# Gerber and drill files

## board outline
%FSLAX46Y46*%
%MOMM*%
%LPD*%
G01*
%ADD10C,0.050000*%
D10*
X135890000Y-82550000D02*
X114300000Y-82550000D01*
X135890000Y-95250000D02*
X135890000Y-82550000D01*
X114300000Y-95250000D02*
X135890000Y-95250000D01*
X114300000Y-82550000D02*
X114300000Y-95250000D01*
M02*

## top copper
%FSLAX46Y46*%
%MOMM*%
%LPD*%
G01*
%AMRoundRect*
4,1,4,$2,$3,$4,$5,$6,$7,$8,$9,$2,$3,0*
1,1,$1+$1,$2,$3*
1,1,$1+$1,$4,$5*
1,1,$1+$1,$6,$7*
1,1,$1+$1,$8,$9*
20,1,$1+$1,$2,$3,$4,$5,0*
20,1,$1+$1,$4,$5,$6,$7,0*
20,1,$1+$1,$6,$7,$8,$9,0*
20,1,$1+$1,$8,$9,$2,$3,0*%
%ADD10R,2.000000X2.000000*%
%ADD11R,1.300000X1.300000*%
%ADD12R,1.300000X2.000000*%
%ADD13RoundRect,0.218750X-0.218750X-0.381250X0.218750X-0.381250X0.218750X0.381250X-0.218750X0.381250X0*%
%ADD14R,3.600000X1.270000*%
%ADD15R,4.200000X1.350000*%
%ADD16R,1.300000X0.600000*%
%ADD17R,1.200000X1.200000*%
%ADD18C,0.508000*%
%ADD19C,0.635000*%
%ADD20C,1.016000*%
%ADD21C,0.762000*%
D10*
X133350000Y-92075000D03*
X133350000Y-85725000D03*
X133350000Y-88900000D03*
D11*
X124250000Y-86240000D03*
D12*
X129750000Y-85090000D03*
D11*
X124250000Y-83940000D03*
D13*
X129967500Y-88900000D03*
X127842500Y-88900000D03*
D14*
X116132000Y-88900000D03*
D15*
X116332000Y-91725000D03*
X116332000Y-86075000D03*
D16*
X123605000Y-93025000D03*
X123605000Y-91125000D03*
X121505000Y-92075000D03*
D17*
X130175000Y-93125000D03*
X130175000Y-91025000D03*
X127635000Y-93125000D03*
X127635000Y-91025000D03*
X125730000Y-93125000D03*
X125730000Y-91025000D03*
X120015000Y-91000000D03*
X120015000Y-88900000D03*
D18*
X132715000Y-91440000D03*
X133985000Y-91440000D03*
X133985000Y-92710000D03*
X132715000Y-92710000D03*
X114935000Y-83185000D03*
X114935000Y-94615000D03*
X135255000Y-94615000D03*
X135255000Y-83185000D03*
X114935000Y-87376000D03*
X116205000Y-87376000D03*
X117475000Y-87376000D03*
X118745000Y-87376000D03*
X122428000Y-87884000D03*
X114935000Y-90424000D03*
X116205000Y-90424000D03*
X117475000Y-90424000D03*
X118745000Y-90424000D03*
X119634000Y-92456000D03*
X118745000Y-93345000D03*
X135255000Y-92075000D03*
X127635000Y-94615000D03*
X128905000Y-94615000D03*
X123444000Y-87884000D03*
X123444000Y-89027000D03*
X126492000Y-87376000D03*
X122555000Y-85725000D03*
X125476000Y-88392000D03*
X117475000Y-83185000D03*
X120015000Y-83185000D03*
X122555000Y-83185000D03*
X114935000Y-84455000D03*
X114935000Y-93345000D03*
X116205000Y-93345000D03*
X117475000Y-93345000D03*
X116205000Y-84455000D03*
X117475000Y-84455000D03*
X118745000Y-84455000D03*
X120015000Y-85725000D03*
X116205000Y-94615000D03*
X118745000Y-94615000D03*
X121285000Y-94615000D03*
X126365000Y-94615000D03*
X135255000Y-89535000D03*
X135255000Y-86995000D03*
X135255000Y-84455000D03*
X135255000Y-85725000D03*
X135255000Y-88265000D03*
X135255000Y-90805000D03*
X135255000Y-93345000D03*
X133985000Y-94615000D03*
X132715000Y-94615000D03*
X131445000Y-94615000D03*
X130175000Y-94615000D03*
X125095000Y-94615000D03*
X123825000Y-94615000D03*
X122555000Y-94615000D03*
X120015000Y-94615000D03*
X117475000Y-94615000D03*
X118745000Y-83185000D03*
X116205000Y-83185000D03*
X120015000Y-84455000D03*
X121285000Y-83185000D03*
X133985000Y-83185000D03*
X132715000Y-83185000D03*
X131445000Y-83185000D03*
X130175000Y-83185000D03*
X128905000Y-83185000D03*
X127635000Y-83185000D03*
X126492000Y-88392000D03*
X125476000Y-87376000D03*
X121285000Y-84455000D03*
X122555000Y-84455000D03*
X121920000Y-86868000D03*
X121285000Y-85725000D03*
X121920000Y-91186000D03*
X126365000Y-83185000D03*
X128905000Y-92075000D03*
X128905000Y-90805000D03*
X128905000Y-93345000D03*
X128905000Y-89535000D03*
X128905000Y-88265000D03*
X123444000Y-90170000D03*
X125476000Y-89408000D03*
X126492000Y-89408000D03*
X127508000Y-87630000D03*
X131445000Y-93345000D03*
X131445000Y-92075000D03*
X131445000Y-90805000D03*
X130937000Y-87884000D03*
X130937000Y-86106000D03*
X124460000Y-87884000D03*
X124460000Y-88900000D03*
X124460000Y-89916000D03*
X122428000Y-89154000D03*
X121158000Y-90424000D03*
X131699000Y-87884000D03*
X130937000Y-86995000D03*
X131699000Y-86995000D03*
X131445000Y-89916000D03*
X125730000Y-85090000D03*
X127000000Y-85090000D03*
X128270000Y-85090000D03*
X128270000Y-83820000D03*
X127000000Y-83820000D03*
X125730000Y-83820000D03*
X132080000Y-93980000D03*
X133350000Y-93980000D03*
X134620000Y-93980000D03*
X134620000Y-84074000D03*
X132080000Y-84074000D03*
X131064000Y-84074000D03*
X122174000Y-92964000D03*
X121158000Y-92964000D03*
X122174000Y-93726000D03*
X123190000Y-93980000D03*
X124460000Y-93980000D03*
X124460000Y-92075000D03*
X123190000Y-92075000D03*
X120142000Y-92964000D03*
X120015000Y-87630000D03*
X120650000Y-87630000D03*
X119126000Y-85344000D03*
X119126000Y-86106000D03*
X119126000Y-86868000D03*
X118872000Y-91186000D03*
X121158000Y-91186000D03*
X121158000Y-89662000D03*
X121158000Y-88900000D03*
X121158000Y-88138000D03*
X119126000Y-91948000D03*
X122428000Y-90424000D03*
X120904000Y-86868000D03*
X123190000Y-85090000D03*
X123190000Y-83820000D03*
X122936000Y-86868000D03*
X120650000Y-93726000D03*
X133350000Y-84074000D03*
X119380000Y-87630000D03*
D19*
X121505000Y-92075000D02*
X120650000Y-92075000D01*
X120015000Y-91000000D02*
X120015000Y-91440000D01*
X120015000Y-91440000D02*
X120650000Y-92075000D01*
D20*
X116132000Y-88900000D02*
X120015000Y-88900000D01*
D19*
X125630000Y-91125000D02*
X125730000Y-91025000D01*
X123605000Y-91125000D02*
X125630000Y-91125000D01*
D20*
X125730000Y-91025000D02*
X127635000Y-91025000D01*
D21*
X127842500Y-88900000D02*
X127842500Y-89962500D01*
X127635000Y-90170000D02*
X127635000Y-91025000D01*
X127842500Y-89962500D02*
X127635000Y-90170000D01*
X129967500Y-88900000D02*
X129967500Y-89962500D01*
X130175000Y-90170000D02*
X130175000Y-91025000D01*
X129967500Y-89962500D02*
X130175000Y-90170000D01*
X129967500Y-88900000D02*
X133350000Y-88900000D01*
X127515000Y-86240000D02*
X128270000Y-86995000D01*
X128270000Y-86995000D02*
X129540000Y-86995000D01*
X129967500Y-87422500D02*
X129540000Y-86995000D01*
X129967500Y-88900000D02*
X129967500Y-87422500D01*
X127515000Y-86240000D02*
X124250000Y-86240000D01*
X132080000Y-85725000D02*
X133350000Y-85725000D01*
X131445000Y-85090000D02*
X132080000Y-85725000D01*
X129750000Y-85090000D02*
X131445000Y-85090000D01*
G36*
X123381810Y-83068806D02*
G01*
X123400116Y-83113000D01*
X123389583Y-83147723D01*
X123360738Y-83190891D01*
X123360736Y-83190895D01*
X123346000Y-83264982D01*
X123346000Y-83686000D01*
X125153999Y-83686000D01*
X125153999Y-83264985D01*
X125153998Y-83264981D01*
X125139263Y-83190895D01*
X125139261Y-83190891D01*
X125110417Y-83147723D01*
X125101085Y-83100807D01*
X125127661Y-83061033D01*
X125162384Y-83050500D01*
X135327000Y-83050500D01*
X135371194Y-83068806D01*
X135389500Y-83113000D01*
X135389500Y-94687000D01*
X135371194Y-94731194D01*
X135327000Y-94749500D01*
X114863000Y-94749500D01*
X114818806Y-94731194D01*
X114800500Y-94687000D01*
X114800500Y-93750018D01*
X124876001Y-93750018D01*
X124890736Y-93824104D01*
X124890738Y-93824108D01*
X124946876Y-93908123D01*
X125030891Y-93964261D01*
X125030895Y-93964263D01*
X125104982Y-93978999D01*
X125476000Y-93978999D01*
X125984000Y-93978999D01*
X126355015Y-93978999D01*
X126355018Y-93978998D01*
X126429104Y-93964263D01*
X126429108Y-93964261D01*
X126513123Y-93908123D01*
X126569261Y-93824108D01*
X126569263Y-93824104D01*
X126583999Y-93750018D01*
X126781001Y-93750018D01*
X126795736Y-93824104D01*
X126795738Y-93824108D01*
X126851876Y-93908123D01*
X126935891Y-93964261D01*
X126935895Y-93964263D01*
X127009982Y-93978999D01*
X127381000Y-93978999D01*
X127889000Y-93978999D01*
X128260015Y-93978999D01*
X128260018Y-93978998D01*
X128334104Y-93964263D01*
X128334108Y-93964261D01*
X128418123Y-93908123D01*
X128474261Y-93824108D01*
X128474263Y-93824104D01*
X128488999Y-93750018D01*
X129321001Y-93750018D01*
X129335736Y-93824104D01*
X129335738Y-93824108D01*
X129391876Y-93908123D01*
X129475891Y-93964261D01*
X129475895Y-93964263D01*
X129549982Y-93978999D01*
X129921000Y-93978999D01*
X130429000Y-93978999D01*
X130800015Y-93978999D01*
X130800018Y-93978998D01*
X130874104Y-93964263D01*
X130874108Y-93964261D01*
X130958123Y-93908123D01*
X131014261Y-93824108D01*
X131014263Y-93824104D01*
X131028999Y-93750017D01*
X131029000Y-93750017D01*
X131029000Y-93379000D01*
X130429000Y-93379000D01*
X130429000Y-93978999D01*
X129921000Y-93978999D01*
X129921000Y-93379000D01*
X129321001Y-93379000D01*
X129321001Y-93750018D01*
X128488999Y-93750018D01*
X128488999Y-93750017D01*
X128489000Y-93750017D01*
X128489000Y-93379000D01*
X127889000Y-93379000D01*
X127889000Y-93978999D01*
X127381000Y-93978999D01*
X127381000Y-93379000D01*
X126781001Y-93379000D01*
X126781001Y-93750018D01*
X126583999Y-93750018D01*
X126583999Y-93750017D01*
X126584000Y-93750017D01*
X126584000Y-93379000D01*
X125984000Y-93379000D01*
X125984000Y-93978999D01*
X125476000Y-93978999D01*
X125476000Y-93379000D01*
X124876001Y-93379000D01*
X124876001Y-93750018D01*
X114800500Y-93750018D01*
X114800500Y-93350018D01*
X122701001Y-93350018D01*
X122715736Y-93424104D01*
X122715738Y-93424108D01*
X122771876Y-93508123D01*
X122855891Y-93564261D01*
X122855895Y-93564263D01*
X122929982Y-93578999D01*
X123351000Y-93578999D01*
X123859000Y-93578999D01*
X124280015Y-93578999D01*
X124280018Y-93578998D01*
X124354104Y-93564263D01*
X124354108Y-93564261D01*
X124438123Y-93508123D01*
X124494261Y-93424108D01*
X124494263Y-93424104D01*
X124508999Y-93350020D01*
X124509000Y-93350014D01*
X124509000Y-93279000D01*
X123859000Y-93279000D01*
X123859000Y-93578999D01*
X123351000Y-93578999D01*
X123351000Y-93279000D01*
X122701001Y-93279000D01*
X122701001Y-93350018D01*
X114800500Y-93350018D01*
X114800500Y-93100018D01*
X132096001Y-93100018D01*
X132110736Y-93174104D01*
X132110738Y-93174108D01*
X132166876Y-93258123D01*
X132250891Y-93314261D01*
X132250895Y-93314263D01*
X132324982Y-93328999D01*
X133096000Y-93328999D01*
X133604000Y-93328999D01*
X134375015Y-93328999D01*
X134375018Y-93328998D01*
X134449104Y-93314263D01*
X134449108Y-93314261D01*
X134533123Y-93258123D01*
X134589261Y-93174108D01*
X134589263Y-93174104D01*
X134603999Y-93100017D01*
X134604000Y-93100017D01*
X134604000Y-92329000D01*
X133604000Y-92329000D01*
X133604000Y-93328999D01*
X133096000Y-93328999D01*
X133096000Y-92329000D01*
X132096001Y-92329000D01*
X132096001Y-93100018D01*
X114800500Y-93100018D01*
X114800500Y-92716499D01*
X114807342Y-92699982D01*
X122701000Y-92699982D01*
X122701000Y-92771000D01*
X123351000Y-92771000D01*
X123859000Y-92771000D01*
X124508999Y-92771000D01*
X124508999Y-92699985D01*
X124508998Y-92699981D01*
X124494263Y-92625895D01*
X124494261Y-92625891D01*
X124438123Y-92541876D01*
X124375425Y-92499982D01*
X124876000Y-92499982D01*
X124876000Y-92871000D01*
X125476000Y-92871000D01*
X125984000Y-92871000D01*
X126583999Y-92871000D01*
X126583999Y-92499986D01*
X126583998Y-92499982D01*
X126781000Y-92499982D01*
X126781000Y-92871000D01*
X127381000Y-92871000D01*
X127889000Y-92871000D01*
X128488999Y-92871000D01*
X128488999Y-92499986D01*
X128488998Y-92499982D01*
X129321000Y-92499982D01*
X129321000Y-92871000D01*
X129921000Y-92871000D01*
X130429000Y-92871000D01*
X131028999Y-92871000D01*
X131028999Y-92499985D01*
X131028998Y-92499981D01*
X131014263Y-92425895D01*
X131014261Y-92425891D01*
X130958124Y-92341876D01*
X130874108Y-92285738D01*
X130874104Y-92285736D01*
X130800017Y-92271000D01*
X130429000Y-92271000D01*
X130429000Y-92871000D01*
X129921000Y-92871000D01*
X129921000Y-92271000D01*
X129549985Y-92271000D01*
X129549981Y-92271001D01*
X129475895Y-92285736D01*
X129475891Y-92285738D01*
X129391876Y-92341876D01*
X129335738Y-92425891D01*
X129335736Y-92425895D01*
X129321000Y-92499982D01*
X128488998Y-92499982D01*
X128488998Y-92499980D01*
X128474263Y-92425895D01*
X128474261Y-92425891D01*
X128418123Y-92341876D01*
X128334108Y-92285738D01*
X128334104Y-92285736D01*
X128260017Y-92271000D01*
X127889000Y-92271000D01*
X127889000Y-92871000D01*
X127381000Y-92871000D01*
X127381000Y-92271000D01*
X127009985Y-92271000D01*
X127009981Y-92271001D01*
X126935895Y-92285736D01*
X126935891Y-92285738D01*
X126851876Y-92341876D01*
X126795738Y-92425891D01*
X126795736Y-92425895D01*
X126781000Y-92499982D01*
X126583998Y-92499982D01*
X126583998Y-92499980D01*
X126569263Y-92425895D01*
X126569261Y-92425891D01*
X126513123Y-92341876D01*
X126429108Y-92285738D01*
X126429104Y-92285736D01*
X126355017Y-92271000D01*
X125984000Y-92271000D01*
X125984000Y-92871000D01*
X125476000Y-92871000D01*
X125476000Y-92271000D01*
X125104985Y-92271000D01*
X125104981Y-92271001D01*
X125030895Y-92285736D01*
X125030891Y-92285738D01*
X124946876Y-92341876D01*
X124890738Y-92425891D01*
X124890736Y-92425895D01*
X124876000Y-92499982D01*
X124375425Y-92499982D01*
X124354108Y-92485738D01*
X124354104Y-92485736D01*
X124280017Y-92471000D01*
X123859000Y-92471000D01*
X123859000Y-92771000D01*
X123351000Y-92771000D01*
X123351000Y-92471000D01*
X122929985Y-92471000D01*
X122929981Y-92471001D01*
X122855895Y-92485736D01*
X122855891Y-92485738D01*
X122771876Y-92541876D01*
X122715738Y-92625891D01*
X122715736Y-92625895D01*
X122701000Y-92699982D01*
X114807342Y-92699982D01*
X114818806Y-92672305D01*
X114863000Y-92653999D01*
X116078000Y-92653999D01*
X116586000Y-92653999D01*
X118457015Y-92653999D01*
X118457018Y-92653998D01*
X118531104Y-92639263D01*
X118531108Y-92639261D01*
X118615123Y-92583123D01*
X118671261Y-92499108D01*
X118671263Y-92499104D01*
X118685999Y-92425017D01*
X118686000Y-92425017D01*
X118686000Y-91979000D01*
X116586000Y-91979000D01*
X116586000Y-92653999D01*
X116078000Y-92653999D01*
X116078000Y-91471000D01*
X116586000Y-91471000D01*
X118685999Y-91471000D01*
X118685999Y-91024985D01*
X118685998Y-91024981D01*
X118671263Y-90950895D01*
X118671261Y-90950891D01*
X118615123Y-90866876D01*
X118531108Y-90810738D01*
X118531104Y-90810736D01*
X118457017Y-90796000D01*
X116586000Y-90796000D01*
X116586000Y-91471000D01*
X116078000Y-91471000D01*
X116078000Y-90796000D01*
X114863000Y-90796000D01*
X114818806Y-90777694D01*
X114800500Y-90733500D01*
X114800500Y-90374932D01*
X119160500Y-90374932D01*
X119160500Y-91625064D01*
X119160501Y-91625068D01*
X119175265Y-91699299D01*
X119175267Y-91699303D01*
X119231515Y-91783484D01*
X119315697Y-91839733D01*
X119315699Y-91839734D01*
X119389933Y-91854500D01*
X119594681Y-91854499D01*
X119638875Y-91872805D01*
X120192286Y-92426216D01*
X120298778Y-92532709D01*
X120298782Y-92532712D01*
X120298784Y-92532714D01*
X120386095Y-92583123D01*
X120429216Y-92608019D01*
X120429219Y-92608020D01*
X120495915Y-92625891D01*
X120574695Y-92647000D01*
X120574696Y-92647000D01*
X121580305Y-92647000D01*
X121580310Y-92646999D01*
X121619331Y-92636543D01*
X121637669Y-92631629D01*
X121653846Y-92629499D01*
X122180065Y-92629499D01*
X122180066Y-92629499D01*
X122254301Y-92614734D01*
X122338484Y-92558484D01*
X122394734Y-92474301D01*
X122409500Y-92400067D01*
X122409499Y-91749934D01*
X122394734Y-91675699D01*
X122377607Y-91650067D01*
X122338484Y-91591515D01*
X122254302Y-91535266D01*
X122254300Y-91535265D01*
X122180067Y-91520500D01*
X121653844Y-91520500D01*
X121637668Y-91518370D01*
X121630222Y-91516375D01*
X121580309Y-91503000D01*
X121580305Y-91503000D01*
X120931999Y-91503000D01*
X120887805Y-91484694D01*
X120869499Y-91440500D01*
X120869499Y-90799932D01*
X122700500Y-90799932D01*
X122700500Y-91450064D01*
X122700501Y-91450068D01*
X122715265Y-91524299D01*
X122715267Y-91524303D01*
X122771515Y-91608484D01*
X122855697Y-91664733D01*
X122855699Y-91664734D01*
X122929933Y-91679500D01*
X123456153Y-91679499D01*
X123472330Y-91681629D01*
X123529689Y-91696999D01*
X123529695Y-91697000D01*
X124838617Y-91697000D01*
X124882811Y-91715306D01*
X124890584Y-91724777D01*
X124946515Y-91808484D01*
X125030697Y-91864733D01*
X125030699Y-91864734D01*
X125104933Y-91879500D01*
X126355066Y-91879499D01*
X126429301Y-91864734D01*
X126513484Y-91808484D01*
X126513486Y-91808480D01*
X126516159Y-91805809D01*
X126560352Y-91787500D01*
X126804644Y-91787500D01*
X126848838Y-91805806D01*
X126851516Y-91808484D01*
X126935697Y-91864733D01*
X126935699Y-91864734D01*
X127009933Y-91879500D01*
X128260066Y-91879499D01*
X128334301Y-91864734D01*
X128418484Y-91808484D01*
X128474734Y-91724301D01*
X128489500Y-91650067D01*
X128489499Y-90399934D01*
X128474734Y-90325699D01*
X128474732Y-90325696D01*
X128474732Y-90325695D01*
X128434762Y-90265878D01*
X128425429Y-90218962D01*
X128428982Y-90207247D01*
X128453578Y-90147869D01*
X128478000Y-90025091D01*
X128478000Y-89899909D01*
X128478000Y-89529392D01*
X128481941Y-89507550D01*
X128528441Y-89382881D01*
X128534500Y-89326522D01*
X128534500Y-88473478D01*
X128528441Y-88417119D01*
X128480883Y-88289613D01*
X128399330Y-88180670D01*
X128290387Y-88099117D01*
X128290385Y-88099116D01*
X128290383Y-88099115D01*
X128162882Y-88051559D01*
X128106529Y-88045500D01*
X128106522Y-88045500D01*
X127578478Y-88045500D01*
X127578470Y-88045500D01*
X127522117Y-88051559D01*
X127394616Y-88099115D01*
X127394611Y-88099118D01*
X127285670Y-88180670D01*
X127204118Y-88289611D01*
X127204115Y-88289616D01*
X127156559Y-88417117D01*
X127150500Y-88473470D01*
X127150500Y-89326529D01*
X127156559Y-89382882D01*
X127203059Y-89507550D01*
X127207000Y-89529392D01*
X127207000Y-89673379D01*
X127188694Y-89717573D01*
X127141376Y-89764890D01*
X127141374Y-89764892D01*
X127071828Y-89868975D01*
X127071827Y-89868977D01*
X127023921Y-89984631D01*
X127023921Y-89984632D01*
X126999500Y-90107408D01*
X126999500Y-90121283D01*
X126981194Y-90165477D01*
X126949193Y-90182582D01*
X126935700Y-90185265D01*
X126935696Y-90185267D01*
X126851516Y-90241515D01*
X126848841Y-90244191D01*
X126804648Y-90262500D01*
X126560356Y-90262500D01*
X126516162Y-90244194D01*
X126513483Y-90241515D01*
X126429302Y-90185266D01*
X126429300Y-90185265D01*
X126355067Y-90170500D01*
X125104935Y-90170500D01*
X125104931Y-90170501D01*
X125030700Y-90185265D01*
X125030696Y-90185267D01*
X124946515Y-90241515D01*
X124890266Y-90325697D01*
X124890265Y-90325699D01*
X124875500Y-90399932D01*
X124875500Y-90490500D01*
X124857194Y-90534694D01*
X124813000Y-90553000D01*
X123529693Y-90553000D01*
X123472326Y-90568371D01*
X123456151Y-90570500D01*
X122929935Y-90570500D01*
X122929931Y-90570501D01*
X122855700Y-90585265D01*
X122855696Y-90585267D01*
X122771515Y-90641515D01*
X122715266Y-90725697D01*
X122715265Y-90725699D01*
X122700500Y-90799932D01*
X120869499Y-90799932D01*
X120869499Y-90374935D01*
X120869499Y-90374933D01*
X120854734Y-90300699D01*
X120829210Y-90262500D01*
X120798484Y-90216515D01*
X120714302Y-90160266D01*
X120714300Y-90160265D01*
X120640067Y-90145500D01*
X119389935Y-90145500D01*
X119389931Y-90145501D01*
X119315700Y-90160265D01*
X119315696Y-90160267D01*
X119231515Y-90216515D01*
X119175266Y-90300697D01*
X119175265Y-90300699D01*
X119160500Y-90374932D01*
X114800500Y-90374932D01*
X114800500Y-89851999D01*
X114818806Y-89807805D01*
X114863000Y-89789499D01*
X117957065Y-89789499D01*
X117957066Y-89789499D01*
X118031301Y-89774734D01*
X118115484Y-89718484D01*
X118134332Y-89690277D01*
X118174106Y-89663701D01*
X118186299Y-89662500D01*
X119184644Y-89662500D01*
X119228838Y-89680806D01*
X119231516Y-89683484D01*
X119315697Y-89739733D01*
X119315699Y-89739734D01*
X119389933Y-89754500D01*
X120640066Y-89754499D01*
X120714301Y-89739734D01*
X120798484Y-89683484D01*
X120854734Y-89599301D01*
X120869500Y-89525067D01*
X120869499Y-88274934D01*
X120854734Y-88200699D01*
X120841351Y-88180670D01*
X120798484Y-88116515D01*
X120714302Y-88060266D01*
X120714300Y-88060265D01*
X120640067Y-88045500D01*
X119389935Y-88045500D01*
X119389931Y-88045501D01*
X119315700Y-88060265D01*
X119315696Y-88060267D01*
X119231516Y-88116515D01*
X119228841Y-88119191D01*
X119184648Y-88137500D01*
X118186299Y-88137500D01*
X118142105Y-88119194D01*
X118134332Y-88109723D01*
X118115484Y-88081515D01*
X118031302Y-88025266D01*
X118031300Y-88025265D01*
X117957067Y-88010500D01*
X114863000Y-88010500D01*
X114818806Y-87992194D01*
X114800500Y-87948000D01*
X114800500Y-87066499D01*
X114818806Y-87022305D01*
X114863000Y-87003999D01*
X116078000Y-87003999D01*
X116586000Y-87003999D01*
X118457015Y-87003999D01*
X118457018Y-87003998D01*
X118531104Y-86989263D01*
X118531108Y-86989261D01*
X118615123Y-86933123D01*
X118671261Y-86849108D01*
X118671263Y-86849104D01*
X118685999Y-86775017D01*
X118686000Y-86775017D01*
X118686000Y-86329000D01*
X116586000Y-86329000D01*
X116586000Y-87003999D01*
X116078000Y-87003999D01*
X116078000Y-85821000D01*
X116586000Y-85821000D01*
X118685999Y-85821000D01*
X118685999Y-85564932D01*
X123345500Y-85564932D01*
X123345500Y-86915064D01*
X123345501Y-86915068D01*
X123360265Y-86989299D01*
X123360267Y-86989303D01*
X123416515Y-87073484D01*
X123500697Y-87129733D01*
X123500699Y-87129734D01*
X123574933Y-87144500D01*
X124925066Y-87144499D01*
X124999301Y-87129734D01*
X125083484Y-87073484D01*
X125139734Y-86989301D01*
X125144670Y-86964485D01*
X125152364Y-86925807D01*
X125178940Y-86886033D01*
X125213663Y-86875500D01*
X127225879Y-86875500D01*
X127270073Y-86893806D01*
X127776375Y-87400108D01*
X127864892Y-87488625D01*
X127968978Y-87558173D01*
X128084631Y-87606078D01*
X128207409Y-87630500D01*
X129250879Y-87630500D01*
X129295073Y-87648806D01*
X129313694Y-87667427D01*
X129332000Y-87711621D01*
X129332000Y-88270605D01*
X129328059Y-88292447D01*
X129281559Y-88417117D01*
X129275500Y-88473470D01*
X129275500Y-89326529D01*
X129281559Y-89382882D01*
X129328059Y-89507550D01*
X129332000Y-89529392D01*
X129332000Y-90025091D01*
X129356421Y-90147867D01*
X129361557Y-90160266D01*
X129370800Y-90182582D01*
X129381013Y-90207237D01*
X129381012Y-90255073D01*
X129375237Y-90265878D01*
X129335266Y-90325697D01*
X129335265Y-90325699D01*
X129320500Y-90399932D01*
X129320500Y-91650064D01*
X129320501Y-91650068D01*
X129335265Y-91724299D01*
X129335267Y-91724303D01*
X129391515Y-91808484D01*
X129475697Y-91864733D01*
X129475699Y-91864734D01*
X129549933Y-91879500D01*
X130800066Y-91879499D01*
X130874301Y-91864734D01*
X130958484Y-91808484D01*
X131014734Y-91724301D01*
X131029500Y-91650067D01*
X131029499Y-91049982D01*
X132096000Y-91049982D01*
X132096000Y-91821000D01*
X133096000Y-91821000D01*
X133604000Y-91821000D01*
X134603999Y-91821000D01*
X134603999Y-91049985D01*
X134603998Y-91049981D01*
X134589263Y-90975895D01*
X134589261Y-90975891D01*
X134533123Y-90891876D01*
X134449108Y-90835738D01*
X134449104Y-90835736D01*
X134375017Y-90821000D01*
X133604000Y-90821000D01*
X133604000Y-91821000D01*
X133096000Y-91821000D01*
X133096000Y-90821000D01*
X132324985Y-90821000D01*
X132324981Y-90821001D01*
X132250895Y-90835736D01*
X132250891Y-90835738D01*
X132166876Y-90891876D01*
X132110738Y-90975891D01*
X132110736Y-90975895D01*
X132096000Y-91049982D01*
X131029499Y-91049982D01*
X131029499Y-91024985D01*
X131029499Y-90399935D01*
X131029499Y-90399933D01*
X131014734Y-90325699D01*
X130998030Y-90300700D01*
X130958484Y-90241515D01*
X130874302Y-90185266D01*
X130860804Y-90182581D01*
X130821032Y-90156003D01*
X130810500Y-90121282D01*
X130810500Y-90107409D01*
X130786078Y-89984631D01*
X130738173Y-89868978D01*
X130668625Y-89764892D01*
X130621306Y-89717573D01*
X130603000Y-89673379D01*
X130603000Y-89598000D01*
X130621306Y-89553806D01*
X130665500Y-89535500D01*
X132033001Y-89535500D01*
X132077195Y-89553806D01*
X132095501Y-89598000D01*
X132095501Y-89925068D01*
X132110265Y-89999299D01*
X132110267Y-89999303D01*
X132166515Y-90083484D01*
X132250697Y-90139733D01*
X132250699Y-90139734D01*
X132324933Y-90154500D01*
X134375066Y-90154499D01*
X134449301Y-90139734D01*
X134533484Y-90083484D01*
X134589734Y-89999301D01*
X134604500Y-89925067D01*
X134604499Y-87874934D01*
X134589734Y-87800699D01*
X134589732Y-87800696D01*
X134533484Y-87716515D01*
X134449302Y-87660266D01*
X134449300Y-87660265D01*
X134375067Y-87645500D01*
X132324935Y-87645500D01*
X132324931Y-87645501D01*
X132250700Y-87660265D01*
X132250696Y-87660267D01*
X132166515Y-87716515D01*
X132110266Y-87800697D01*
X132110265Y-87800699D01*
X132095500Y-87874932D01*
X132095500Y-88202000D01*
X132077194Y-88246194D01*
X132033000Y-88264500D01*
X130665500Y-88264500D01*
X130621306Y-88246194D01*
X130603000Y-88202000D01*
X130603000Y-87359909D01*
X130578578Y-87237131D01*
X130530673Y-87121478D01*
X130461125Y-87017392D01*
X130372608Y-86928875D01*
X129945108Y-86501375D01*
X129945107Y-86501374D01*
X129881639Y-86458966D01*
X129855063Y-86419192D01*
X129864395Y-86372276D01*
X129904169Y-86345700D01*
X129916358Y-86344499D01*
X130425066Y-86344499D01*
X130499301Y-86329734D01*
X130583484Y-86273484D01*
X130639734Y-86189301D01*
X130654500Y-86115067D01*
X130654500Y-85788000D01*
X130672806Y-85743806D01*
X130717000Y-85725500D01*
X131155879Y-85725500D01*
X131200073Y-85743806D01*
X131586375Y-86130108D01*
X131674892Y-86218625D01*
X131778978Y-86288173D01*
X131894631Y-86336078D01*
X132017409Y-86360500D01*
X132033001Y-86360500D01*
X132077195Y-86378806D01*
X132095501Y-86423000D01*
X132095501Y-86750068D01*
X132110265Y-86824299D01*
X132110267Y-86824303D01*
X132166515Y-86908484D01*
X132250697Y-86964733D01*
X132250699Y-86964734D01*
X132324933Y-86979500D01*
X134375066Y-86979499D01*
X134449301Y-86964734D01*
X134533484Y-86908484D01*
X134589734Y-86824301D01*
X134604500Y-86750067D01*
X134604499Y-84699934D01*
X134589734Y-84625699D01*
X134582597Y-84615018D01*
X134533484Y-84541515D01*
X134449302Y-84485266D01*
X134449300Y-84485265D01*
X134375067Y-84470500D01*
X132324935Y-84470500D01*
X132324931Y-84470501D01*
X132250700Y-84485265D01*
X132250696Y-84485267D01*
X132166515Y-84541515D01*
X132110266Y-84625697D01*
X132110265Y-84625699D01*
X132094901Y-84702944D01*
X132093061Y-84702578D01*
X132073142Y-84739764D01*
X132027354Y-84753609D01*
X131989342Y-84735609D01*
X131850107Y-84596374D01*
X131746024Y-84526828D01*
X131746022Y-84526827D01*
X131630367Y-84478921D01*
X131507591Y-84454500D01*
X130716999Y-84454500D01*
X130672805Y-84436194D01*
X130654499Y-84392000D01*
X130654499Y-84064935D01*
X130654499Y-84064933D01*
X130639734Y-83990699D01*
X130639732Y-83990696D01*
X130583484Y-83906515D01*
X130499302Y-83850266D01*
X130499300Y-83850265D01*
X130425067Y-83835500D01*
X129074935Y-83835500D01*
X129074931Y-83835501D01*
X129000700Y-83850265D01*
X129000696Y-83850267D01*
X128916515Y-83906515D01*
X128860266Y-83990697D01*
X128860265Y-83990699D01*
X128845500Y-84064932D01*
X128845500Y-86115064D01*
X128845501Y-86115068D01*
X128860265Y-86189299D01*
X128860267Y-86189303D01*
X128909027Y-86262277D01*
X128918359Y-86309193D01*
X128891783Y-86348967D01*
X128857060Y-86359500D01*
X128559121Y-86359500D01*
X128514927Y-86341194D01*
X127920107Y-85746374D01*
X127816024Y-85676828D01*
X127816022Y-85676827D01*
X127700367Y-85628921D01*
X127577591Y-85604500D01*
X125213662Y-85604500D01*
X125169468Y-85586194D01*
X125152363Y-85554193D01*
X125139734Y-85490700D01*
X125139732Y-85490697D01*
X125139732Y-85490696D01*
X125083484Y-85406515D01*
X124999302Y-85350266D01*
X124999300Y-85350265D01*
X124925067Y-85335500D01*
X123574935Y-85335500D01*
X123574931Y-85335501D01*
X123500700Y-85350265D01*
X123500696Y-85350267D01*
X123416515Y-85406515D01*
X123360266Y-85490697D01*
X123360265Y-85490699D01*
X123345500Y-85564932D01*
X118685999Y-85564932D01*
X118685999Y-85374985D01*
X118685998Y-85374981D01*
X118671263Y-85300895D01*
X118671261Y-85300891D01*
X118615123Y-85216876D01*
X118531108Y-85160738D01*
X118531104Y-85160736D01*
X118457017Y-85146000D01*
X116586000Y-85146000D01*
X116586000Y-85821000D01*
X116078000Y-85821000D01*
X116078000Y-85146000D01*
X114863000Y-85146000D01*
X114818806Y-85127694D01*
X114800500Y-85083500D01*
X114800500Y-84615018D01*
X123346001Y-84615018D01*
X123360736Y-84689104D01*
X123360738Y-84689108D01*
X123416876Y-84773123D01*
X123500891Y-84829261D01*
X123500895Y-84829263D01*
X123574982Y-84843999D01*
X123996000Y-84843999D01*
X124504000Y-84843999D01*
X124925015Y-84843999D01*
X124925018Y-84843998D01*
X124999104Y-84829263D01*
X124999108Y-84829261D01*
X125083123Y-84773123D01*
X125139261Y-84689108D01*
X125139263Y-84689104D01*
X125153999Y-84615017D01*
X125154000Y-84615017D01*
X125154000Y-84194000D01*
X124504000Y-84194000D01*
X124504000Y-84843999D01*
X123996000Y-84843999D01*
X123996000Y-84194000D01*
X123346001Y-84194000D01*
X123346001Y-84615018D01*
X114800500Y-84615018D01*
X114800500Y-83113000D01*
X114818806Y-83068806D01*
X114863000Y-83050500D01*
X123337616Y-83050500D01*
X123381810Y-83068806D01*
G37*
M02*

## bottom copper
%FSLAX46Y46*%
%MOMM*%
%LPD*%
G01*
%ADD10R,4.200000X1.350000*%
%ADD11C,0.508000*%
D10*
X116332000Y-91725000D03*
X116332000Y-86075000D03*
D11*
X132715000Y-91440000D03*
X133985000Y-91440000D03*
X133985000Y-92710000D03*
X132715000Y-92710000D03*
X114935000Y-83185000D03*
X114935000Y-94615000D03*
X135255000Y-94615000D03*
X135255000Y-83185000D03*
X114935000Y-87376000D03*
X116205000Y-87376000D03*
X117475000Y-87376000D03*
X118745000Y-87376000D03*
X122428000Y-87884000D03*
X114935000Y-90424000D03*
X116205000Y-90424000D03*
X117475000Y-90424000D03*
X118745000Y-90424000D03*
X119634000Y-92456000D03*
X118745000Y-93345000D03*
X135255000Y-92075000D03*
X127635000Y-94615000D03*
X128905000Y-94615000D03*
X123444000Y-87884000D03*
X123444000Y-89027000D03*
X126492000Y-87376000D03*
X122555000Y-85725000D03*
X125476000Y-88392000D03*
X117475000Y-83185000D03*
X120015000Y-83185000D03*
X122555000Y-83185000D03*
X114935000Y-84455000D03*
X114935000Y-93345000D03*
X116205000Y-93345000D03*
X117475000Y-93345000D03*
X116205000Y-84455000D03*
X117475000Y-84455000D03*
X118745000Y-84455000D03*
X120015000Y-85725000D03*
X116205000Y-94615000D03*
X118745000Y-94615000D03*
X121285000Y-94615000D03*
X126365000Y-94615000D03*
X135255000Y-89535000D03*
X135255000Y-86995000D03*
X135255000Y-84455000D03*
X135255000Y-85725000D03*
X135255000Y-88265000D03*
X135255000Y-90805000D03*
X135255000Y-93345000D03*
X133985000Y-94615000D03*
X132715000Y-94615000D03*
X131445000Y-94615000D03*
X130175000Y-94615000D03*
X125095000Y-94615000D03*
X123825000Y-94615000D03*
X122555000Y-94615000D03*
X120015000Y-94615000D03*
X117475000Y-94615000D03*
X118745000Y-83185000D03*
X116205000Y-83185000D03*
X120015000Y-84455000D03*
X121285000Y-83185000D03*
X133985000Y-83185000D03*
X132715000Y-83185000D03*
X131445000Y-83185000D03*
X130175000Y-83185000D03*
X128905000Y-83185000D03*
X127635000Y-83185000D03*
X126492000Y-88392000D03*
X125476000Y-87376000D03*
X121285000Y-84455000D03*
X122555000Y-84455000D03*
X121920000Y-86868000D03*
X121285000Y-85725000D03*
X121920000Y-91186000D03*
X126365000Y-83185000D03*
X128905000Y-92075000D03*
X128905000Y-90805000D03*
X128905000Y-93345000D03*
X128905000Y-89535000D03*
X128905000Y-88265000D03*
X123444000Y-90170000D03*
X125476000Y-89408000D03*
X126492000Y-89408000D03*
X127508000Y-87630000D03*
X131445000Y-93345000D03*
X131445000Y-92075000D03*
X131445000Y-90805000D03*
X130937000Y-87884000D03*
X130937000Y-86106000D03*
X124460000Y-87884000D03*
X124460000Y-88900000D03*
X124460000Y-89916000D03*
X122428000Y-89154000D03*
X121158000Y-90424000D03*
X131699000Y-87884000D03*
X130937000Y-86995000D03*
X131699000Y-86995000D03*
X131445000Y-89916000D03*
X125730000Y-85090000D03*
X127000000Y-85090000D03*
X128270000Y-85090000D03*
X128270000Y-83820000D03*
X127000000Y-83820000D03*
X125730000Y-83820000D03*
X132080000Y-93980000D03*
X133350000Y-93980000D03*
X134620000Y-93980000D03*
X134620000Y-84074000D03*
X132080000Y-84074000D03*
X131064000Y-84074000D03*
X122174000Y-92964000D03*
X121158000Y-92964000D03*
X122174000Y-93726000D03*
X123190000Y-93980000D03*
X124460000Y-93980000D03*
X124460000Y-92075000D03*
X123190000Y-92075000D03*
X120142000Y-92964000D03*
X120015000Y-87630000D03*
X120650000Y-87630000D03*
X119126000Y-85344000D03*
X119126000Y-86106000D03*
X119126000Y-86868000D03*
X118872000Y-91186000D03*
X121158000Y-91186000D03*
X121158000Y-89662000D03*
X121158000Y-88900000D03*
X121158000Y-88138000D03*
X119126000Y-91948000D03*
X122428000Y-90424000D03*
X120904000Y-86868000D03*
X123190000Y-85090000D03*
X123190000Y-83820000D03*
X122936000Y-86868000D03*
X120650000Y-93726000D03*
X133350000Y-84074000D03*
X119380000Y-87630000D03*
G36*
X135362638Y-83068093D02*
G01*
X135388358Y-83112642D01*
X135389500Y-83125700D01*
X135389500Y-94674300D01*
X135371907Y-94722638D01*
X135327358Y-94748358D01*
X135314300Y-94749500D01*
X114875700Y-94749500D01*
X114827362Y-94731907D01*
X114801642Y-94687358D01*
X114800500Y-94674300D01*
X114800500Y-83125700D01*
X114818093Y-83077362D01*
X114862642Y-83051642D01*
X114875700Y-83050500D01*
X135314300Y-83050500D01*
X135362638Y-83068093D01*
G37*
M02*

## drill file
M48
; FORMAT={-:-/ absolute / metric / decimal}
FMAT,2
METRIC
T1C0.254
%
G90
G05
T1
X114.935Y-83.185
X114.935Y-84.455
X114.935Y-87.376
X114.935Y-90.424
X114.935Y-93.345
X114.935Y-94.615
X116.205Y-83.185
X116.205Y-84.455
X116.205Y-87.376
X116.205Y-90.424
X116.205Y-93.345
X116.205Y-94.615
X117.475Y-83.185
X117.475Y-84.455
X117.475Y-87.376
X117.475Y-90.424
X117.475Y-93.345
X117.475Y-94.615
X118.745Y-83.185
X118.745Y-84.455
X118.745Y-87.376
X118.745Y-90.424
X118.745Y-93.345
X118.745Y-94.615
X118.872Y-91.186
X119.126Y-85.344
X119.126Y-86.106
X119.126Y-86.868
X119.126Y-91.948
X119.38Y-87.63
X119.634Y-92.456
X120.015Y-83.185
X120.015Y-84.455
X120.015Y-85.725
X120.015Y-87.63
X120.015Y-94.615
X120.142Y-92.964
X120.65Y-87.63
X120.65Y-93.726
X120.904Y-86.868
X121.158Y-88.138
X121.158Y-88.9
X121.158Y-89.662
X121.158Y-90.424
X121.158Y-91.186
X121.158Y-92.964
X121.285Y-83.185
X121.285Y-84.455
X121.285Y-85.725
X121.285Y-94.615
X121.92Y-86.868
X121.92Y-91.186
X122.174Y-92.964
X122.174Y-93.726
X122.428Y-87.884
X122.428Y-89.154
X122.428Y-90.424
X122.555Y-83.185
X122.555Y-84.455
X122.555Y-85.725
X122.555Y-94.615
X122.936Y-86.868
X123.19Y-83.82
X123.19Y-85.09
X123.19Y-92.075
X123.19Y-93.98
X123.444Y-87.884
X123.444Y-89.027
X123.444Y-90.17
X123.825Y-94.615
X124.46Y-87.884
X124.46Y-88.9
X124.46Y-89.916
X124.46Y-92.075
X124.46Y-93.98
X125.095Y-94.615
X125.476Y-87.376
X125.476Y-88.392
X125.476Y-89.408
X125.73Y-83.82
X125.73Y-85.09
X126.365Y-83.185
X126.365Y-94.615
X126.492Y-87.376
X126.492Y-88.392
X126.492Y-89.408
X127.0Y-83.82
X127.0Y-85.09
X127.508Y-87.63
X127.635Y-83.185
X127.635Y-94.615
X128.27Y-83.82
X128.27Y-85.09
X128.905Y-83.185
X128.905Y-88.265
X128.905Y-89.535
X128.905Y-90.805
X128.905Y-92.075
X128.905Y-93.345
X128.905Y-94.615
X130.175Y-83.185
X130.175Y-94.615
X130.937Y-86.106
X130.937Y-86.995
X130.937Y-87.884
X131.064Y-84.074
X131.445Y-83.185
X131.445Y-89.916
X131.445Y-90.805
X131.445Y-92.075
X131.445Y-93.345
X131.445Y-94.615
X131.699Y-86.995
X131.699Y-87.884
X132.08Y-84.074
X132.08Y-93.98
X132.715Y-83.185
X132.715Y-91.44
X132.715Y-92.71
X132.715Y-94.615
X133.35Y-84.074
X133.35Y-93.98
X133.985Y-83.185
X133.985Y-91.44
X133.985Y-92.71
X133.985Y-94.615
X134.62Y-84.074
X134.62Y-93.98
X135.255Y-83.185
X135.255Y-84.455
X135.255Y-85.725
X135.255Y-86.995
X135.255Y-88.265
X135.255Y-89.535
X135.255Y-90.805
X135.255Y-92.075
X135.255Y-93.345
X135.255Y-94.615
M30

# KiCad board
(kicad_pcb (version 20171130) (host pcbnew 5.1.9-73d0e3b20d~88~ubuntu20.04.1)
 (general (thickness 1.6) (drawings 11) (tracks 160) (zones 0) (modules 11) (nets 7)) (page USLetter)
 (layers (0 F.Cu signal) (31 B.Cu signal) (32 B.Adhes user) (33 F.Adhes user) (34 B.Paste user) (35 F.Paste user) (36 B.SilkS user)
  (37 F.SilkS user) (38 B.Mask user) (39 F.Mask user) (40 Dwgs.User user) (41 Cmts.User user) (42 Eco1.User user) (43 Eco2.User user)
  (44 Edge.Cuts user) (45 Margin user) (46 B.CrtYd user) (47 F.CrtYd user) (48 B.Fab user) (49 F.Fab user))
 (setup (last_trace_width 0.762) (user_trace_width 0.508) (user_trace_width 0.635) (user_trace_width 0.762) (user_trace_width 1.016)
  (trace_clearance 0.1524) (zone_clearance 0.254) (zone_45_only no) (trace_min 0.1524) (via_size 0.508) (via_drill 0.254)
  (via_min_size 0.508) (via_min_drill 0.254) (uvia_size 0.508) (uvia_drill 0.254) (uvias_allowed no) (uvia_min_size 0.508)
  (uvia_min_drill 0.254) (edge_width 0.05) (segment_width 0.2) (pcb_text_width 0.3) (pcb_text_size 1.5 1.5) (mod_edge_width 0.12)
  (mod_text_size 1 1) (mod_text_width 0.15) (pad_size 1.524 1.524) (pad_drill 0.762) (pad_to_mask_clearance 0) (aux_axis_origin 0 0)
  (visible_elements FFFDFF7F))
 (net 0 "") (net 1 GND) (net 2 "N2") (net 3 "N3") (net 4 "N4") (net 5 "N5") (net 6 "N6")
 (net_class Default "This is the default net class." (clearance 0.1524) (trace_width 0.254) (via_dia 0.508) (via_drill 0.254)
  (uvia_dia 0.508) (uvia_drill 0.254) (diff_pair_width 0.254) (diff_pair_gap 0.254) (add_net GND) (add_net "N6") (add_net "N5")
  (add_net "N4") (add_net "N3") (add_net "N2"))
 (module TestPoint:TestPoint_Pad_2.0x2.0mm (layer F.Cu) (at 133.35 92.075 270)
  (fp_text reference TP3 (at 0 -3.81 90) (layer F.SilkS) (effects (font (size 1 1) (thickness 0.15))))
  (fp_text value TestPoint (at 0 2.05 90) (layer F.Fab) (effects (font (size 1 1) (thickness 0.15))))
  (pad 1 smd rect (at 0 0 270) (size 2 2) (layers F.Cu F.Mask) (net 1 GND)))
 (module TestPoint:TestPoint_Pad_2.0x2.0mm (layer F.Cu) (at 133.35 85.725 270)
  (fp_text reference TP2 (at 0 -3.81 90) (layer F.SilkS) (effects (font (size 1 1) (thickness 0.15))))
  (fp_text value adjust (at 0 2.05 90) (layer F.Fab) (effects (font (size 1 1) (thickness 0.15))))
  (pad 1 smd rect (at 0 0 270) (size 2 2) (layers F.Cu F.Mask) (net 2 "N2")))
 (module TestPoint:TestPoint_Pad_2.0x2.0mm (layer F.Cu) (at 133.35 88.9 270)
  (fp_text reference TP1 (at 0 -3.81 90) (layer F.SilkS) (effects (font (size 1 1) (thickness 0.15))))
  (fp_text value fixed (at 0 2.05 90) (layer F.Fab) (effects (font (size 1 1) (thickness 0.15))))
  (pad 1 smd rect (at 0 0 270) (size 2 2) (layers F.Cu F.Mask) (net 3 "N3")))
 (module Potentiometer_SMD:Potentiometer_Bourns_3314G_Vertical (layer F.Cu) (at 127 85.09 90)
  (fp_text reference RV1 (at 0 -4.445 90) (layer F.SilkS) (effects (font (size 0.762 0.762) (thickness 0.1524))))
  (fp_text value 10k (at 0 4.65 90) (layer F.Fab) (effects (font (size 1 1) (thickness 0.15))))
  (pad 3 smd rect (at -1.15 -2.75 90) (size 1.3 1.3) (layers F.Cu F.Paste F.Mask) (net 3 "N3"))
  (pad 2 smd rect (at 0 2.75 90) (size 2 1.3) (layers F.Cu F.Paste F.Mask) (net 2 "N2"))
  (pad 1 smd rect (at 1.15 -2.75 90) (size 1.3 1.3) (layers F.Cu F.Paste F.Mask) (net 1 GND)))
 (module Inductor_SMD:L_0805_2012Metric (layer F.Cu) (at 128.905 88.9)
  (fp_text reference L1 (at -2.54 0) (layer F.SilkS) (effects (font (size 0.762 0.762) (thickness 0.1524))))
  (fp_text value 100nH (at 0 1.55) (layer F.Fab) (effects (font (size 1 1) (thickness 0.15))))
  (pad 2 smd roundrect (at 1.0625 0) (size 0.875 1.2) (layers F.Cu F.Paste F.Mask) (roundrect_rratio 0.25) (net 3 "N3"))
  (pad 1 smd roundrect (at -1.0625 0) (size 0.875 1.2) (layers F.Cu F.Paste F.Mask) (roundrect_rratio 0.25) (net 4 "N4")))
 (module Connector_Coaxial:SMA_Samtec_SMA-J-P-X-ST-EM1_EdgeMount (layer F.Cu) (at 116.332 88.9 270)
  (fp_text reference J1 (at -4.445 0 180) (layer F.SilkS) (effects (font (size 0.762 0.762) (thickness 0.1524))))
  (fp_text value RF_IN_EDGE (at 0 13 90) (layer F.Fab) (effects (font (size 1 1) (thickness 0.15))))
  (pad 1 smd rect (at 0 0.2 270) (size 1.27 3.6) (layers F.Cu F.Paste F.Mask) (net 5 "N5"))
  (pad 2 smd rect (at 2.825 0 270) (size 1.35 4.2) (layers F.Cu F.Paste F.Mask) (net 1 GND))
  (pad 2 smd rect (at -2.825 0 270) (size 1.35 4.2) (layers F.Cu F.Paste F.Mask) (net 1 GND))
  (pad 2 smd rect (at 2.825 0 270) (size 1.35 4.2) (layers B.Cu B.Paste B.Mask) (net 1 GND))
  (pad 2 smd rect (at -2.825 0 270) (size 1.35 4.2) (layers B.Cu B.Paste B.Mask) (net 1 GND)))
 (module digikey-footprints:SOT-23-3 (layer F.Cu) (at 122.555 92.075 180)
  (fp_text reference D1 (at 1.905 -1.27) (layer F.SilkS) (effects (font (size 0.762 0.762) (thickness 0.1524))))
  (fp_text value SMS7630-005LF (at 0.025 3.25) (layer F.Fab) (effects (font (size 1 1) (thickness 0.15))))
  (pad 1 smd rect (at -1.05 -0.95 180) (size 1.3 0.6) (layers F.Cu F.Paste F.Mask) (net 1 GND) (solder_mask_margin 0.07))
  (pad 2 smd rect (at -1.05 0.95 180) (size 1.3 0.6) (layers F.Cu F.Paste F.Mask) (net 4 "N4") (solder_mask_margin 0.07))
  (pad 3 smd rect (at 1.05 0 180) (size 1.3 0.6) (layers F.Cu F.Paste F.Mask) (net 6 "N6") (solder_mask_margin 0.07)))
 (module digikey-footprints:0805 (layer F.Cu) (at 130.175 92.075 90)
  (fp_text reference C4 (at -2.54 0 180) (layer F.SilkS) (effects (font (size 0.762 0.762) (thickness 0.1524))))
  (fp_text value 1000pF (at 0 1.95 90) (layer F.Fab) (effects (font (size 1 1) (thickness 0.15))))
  (pad 1 smd rect (at -1.05 0 90) (size 1.2 1.2) (layers F.Cu F.Paste F.Mask) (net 1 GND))
  (pad 2 smd rect (at 1.05 0 90) (size 1.2 1.2) (layers F.Cu F.Paste F.Mask) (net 3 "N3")))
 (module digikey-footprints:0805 (layer F.Cu) (at 127.635 92.075 90)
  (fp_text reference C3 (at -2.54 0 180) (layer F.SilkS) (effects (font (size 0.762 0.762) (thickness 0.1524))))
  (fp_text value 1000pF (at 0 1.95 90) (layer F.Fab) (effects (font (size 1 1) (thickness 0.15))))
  (pad 1 smd rect (at -1.05 0 90) (size 1.2 1.2) (layers F.Cu F.Paste F.Mask) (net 1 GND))
  (pad 2 smd rect (at 1.05 0 90) (size 1.2 1.2) (layers F.Cu F.Paste F.Mask) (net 4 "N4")))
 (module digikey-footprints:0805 (layer F.Cu) (at 125.73 92.075 90)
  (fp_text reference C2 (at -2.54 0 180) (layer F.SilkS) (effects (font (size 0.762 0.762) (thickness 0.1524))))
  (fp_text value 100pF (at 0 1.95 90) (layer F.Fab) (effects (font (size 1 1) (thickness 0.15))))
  (pad 1 smd rect (at -1.05 0 90) (size 1.2 1.2) (layers F.Cu F.Paste F.Mask) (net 1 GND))
  (pad 2 smd rect (at 1.05 0 90) (size 1.2 1.2) (layers F.Cu F.Paste F.Mask) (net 4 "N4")))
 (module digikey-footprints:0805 (layer F.Cu) (at 120.015 89.95 90)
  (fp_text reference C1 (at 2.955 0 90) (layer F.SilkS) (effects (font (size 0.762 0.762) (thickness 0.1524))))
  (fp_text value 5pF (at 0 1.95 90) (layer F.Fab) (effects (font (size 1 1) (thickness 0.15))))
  (pad 1 smd rect (at -1.05 0 90) (size 1.2 1.2) (layers F.Cu F.Paste F.Mask) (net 6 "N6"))
  (pad 2 smd rect (at 1.05 0 90) (size 1.2 1.2) (layers F.Cu F.Paste F.Mask) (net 5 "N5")))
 (gr_line (start 135.89 82.55) (end 114.3 82.55) (layer Edge.Cuts) (width 0.05))
 (gr_line (start 135.89 95.25) (end 135.89 82.55) (layer Edge.Cuts) (width 0.05))
 (gr_line (start 114.3 95.25) (end 135.89 95.25) (layer Edge.Cuts) (width 0.05))
 (gr_line (start 114.3 82.55) (end 114.3 95.25) (layer Edge.Cuts) (width 0.05))
 (via (at 132.715 91.44) (size 0.508) (drill 0.254) (layers F.Cu B.Cu) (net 1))
 (via (at 133.985 91.44) (size 0.508) (drill 0.254) (layers F.Cu B.Cu) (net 1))
 (via (at 133.985 92.71) (size 0.508) (drill 0.254) (layers F.Cu B.Cu) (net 1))
 (via (at 132.715 92.71) (size 0.508) (drill 0.254) (layers F.Cu B.Cu) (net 1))
 (segment (start 121.505 92.075) (end 120.65 92.075) (width 0.635) (layer F.Cu) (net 6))
 (segment (start 120.015 91) (end 120.015 91.44) (width 0.635) (layer F.Cu) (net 6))
 (segment (start 120.015 91.44) (end 120.65 92.075) (width 0.635) (layer F.Cu) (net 6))
 (segment (start 116.132 88.9) (end 120.015 88.9) (width 1.016) (layer F.Cu) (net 5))
 (via (at 114.935 83.185) (size 0.508) (drill 0.254) (layers F.Cu B.Cu) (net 1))
 (via (at 114.935 94.615) (size 0.508) (drill 0.254) (layers F.Cu B.Cu) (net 1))
 (via (at 135.255 94.615) (size 0.508) (drill 0.254) (layers F.Cu B.Cu) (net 1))
 (via (at 135.255 83.185) (size 0.508) (drill 0.254) (layers F.Cu B.Cu) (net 1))
 (via (at 114.935 87.376) (size 0.508) (drill 0.254) (layers F.Cu B.Cu) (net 1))
 (via (at 116.205 87.376) (size 0.508) (drill 0.254) (layers F.Cu B.Cu) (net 1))
 (via (at 117.475 87.376) (size 0.508) (drill 0.254) (layers F.Cu B.Cu) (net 1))
 (via (at 118.745 87.376) (size 0.508) (drill 0.254) (layers F.Cu B.Cu) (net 1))
 (via (at 122.428 87.884) (size 0.508) (drill 0.254) (layers F.Cu B.Cu) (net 1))
 (via (at 114.935 90.424) (size 0.508) (drill 0.254) (layers F.Cu B.Cu) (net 1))
 (via (at 116.205 90.424) (size 0.508) (drill 0.254) (layers F.Cu B.Cu) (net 1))
 (via (at 117.475 90.424) (size 0.508) (drill 0.254) (layers F.Cu B.Cu) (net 1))
 (via (at 118.745 90.424) (size 0.508) (drill 0.254) (layers F.Cu B.Cu) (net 1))
 (via (at 119.634 92.456) (size 0.508) (drill 0.254) (layers F.Cu B.Cu) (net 1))
 (via (at 118.745 93.345) (size 0.508) (drill 0.254) (layers F.Cu B.Cu) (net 1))
 (via (at 135.255 92.075) (size 0.508) (drill 0.254) (layers F.Cu B.Cu) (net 1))
 (via (at 127.635 94.615) (size 0.508) (drill 0.254) (layers F.Cu B.Cu) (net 1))
 (via (at 128.905 94.615) (size 0.508) (drill 0.254) (layers F.Cu B.Cu) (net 1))
 (via (at 123.444 87.884) (size 0.508) (drill 0.254) (layers F.Cu B.Cu) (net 1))
 (via (at 123.444 89.027) (size 0.508) (drill 0.254) (layers F.Cu B.Cu) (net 1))
 (via (at 126.492 87.376) (size 0.508) (drill 0.254) (layers F.Cu B.Cu) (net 1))
 (via (at 122.555 85.725) (size 0.508) (drill 0.254) (layers F.Cu B.Cu) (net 1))
 (via (at 125.476 88.392) (size 0.508) (drill 0.254) (layers F.Cu B.Cu) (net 1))
 (via (at 117.475 83.185) (size 0.508) (drill 0.254) (layers F.Cu B.Cu) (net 1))
 (via (at 120.015 83.185) (size 0.508) (drill 0.254) (layers F.Cu B.Cu) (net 1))
 (via (at 122.555 83.185) (size 0.508) (drill 0.254) (layers F.Cu B.Cu) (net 1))
 (via (at 114.935 84.455) (size 0.508) (drill 0.254) (layers F.Cu B.Cu) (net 1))
 (via (at 114.935 93.345) (size 0.508) (drill 0.254) (layers F.Cu B.Cu) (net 1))
 (via (at 116.205 93.345) (size 0.508) (drill 0.254) (layers F.Cu B.Cu) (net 1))
 (via (at 117.475 93.345) (size 0.508) (drill 0.254) (layers F.Cu B.Cu) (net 1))
 (via (at 116.205 84.455) (size 0.508) (drill 0.254) (layers F.Cu B.Cu) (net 1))
 (via (at 117.475 84.455) (size 0.508) (drill 0.254) (layers F.Cu B.Cu) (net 1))
 (via (at 118.745 84.455) (size 0.508) (drill 0.254) (layers F.Cu B.Cu) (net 1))
 (via (at 120.015 85.725) (size 0.508) (drill 0.254) (layers F.Cu B.Cu) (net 1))
 (via (at 116.205 94.615) (size 0.508) (drill 0.254) (layers F.Cu B.Cu) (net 1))
 (via (at 118.745 94.615) (size 0.508) (drill 0.254) (layers F.Cu B.Cu) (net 1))
 (via (at 121.285 94.615) (size 0.508) (drill 0.254) (layers F.Cu B.Cu) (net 1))
 (via (at 126.365 94.615) (size 0.508) (drill 0.254) (layers F.Cu B.Cu) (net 1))
 (via (at 135.255 89.535) (size 0.508) (drill 0.254) (layers F.Cu B.Cu) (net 1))
 (via (at 135.255 86.995) (size 0.508) (drill 0.254) (layers F.Cu B.Cu) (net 1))
 (via (at 135.255 84.455) (size 0.508) (drill 0.254) (layers F.Cu B.Cu) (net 1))
 (via (at 135.255 85.725) (size 0.508) (drill 0.254) (layers F.Cu B.Cu) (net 1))
 (via (at 135.255 88.265) (size 0.508) (drill 0.254) (layers F.Cu B.Cu) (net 1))
 (via (at 135.255 90.805) (size 0.508) (drill 0.254) (layers F.Cu B.Cu) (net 1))
 (via (at 135.255 93.345) (size 0.508) (drill 0.254) (layers F.Cu B.Cu) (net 1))
 (via (at 133.985 94.615) (size 0.508) (drill 0.254) (layers F.Cu B.Cu) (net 1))
 (via (at 132.715 94.615) (size 0.508) (drill 0.254) (layers F.Cu B.Cu) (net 1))
 (via (at 131.445 94.615) (size 0.508) (drill 0.254) (layers F.Cu B.Cu) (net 1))
 (via (at 130.175 94.615) (size 0.508) (drill 0.254) (layers F.Cu B.Cu) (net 1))
 (via (at 125.095 94.615) (size 0.508) (drill 0.254) (layers F.Cu B.Cu) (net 1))
 (via (at 123.825 94.615) (size 0.508) (drill 0.254) (layers F.Cu B.Cu) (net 1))
 (via (at 122.555 94.615) (size 0.508) (drill 0.254) (layers F.Cu B.Cu) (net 1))
 (via (at 120.015 94.615) (size 0.508) (drill 0.254) (layers F.Cu B.Cu) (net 1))
 (via (at 117.475 94.615) (size 0.508) (drill 0.254) (layers F.Cu B.Cu) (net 1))
 (via (at 118.745 83.185) (size 0.508) (drill 0.254) (layers F.Cu B.Cu) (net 1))
 (via (at 116.205 83.185) (size 0.508) (drill 0.254) (layers F.Cu B.Cu) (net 1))
 (via (at 120.015 84.455) (size 0.508) (drill 0.254) (layers F.Cu B.Cu) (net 1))
 (via (at 121.285 83.185) (size 0.508) (drill 0.254) (layers F.Cu B.Cu) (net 1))
 (via (at 133.985 83.185) (size 0.508) (drill 0.254) (layers F.Cu B.Cu) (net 1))
 (via (at 132.715 83.185) (size 0.508) (drill 0.254) (layers F.Cu B.Cu) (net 1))
 (via (at 131.445 83.185) (size 0.508) (drill 0.254) (layers F.Cu B.Cu) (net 1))
 (via (at 130.175 83.185) (size 0.508) (drill 0.254) (layers F.Cu B.Cu) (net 1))
 (via (at 128.905 83.185) (size 0.508) (drill 0.254) (layers F.Cu B.Cu) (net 1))
 (via (at 127.635 83.185) (size 0.508) (drill 0.254) (layers F.Cu B.Cu) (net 1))
 (via (at 126.492 88.392) (size 0.508) (drill 0.254) (layers F.Cu B.Cu) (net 1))
 (via (at 125.476 87.376) (size 0.508) (drill 0.254) (layers F.Cu B.Cu) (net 1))
 (via (at 121.285 84.455) (size 0.508) (drill 0.254) (layers F.Cu B.Cu) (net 1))
 (via (at 122.555 84.455) (size 0.508) (drill 0.254) (layers F.Cu B.Cu) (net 1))
 (via (at 121.92 86.868) (size 0.508) (drill 0.254) (layers F.Cu B.Cu) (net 1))
 (via (at 121.285 85.725) (size 0.508) (drill 0.254) (layers F.Cu B.Cu) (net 1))
 (via (at 121.92 91.186) (size 0.508) (drill 0.254) (layers F.Cu B.Cu) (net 1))
 (via (at 126.365 83.185) (size 0.508) (drill 0.254) (layers F.Cu B.Cu) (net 1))
 (via (at 128.905 92.075) (size 0.508) (drill 0.254) (layers F.Cu B.Cu) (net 1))
 (via (at 128.905 90.805) (size 0.508) (drill 0.254) (layers F.Cu B.Cu) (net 1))
 (via (at 128.905 93.345) (size 0.508) (drill 0.254) (layers F.Cu B.Cu) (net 1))
 (via (at 128.905 89.535) (size 0.508) (drill 0.254) (layers F.Cu B.Cu) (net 1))
 (via (at 128.905 88.265) (size 0.508) (drill 0.254) (layers F.Cu B.Cu) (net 1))
 (via (at 123.444 90.17) (size 0.508) (drill 0.254) (layers F.Cu B.Cu) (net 1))
 (via (at 125.476 89.408) (size 0.508) (drill 0.254) (layers F.Cu B.Cu) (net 1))
 (via (at 126.492 89.408) (size 0.508) (drill 0.254) (layers F.Cu B.Cu) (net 1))
 (via (at 127.508 87.63) (size 0.508) (drill 0.254) (layers F.Cu B.Cu) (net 1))
 (via (at 131.445 93.345) (size 0.508) (drill 0.254) (layers F.Cu B.Cu) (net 1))
 (via (at 131.445 92.075) (size 0.508) (drill 0.254) (layers F.Cu B.Cu) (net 1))
 (via (at 131.445 90.805) (size 0.508) (drill 0.254) (layers F.Cu B.Cu) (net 1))
 (via (at 130.937 87.884) (size 0.508) (drill 0.254) (layers F.Cu B.Cu) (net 1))
 (via (at 130.937 86.106) (size 0.508) (drill 0.254) (layers F.Cu B.Cu) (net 1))
 (via (at 124.46 87.884) (size 0.508) (drill 0.254) (layers F.Cu B.Cu) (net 1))
 (via (at 124.46 88.9) (size 0.508) (drill 0.254) (layers F.Cu B.Cu) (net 1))
 (via (at 124.46 89.916) (size 0.508) (drill 0.254) (layers F.Cu B.Cu) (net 1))
 (via (at 122.428 89.154) (size 0.508) (drill 0.254) (layers F.Cu B.Cu) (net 1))
 (via (at 121.158 90.424) (size 0.508) (drill 0.254) (layers F.Cu B.Cu) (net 1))
 (via (at 131.699 87.884) (size 0.508) (drill 0.254) (layers F.Cu B.Cu) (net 1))
 (via (at 130.937 86.995) (size 0.508) (drill 0.254) (layers F.Cu B.Cu) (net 1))
 (via (at 131.699 86.995) (size 0.508) (drill 0.254) (layers F.Cu B.Cu) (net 1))
 (via (at 131.445 89.916) (size 0.508) (drill 0.254) (layers F.Cu B.Cu) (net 1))
 (via (at 125.73 85.09) (size 0.508) (drill 0.254) (layers F.Cu B.Cu) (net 1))
 (via (at 127 85.09) (size 0.508) (drill 0.254) (layers F.Cu B.Cu) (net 1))
 (via (at 128.27 85.09) (size 0.508) (drill 0.254) (layers F.Cu B.Cu) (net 1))
 (via (at 128.27 83.82) (size 0.508) (drill 0.254) (layers F.Cu B.Cu) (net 1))
 (via (at 127 83.82) (size 0.508) (drill 0.254) (layers F.Cu B.Cu) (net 1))
 (via (at 125.73 83.82) (size 0.508) (drill 0.254) (layers F.Cu B.Cu) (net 1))
 (via (at 132.08 93.98) (size 0.508) (drill 0.254) (layers F.Cu B.Cu) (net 1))
 (via (at 133.35 93.98) (size 0.508) (drill 0.254) (layers F.Cu B.Cu) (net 1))
 (via (at 134.62 93.98) (size 0.508) (drill 0.254) (layers F.Cu B.Cu) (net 1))
 (via (at 134.62 84.074) (size 0.508) (drill 0.254) (layers F.Cu B.Cu) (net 1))
 (via (at 132.08 84.074) (size 0.508) (drill 0.254) (layers F.Cu B.Cu) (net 1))
 (via (at 131.064 84.074) (size 0.508) (drill 0.254) (layers F.Cu B.Cu) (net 1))
 (via (at 122.174 92.964) (size 0.508) (drill 0.254) (layers F.Cu B.Cu) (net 1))
 (via (at 121.158 92.964) (size 0.508) (drill 0.254) (layers F.Cu B.Cu) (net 1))
 (via (at 122.174 93.726) (size 0.508) (drill 0.254) (layers F.Cu B.Cu) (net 1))
 (via (at 123.19 93.98) (size 0.508) (drill 0.254) (layers F.Cu B.Cu) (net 1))
 (via (at 124.46 93.98) (size 0.508) (drill 0.254) (layers F.Cu B.Cu) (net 1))
 (via (at 124.46 92.075) (size 0.508) (drill 0.254) (layers F.Cu B.Cu) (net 1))
 (via (at 123.19 92.075) (size 0.508) (drill 0.254) (layers F.Cu B.Cu) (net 1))
 (via (at 120.142 92.964) (size 0.508) (drill 0.254) (layers F.Cu B.Cu) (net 1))
 (via (at 120.015 87.63) (size 0.508) (drill 0.254) (layers F.Cu B.Cu) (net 1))
 (via (at 120.65 87.63) (size 0.508) (drill 0.254) (layers F.Cu B.Cu) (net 1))
 (via (at 119.126 85.344) (size 0.508) (drill 0.254) (layers F.Cu B.Cu) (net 1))
 (via (at 119.126 86.106) (size 0.508) (drill 0.254) (layers F.Cu B.Cu) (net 1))
 (via (at 119.126 86.868) (size 0.508) (drill 0.254) (layers F.Cu B.Cu) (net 1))
 (via (at 118.872 91.186) (size 0.508) (drill 0.254) (layers F.Cu B.Cu) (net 1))
 (via (at 121.158 91.186) (size 0.508) (drill 0.254) (layers F.Cu B.Cu) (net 1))
 (via (at 121.158 89.662) (size 0.508) (drill 0.254) (layers F.Cu B.Cu) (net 1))
 (via (at 121.158 88.9) (size 0.508) (drill 0.254) (layers F.Cu B.Cu) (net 1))
 (via (at 121.158 88.138) (size 0.508) (drill 0.254) (layers F.Cu B.Cu) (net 1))
 (via (at 119.126 91.948) (size 0.508) (drill 0.254) (layers F.Cu B.Cu) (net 1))
 (via (at 122.428 90.424) (size 0.508) (drill 0.254) (layers F.Cu B.Cu) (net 1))
 (via (at 120.904 86.868) (size 0.508) (drill 0.254) (layers F.Cu B.Cu) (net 1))
 (via (at 123.19 85.09) (size 0.508) (drill 0.254) (layers F.Cu B.Cu) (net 1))
 (via (at 123.19 83.82) (size 0.508) (drill 0.254) (layers F.Cu B.Cu) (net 1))
 (via (at 122.936 86.868) (size 0.508) (drill 0.254) (layers F.Cu B.Cu) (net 1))
 (via (at 120.65 93.726) (size 0.508) (drill 0.254) (layers F.Cu B.Cu) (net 1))
 (via (at 133.35 84.074) (size 0.508) (drill 0.254) (layers F.Cu B.Cu) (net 1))
 (via (at 119.38 87.63) (size 0.508) (drill 0.254) (layers F.Cu B.Cu) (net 1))
 (segment (start 125.63 91.125) (end 125.73 91.025) (width 0.635) (layer F.Cu) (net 4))
 (segment (start 123.605 91.125) (end 125.63 91.125) (width 0.635) (layer F.Cu) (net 4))
 (segment (start 125.73 91.025) (end 127.635 91.025) (width 1.016) (layer F.Cu) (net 4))
 (segment (start 127.8425 88.9) (end 127.8425 89.9625) (width 0.762) (layer F.Cu) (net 4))
 (segment (start 127.635 90.17) (end 127.635 91.025) (width 0.762) (layer F.Cu) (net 4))
 (segment (start 127.8425 89.9625) (end 127.635 90.17) (width 0.762) (layer F.Cu) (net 4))
 (segment (start 129.9675 88.9) (end 129.9675 89.9625) (width 0.762) (layer F.Cu) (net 3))
 (segment (start 130.175 90.17) (end 130.175 91.025) (width 0.762) (layer F.Cu) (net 3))
 (segment (start 129.9675 89.9625) (end 130.175 90.17) (width 0.762) (layer F.Cu) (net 3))
 (segment (start 129.9675 88.9) (end 133.35 88.9) (width 0.762) (layer F.Cu) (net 3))
 (segment (start 127.515 86.24) (end 128.27 86.995) (width 0.762) (layer F.Cu) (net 3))
 (segment (start 128.27 86.995) (end 129.54 86.995) (width 0.762) (layer F.Cu) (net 3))
 (segment (start 129.9675 87.4225) (end 129.54 86.995) (width 0.762) (layer F.Cu) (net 3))
 (segment (start 129.9675 88.9) (end 129.9675 87.4225) (width 0.762) (layer F.Cu) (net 3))
 (segment (start 127.515 86.24) (end 124.25 86.24) (width 0.762) (layer F.Cu) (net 3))
 (segment (start 132.08 85.725) (end 133.35 85.725) (width 0.762) (layer F.Cu) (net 2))
 (segment (start 131.445 85.09) (end 132.08 85.725) (width 0.762) (layer F.Cu) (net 2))
 (segment (start 129.75 85.09) (end 131.445 85.09) (width 0.762) (layer F.Cu) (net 2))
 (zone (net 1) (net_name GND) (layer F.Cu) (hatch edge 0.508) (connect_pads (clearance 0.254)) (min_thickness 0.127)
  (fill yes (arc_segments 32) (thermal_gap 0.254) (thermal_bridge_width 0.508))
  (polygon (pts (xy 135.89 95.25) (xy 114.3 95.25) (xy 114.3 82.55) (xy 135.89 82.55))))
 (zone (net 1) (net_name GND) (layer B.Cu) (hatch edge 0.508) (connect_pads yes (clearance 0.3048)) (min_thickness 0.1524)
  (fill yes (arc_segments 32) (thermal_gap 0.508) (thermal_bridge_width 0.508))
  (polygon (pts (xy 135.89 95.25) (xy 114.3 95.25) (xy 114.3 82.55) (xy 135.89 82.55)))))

